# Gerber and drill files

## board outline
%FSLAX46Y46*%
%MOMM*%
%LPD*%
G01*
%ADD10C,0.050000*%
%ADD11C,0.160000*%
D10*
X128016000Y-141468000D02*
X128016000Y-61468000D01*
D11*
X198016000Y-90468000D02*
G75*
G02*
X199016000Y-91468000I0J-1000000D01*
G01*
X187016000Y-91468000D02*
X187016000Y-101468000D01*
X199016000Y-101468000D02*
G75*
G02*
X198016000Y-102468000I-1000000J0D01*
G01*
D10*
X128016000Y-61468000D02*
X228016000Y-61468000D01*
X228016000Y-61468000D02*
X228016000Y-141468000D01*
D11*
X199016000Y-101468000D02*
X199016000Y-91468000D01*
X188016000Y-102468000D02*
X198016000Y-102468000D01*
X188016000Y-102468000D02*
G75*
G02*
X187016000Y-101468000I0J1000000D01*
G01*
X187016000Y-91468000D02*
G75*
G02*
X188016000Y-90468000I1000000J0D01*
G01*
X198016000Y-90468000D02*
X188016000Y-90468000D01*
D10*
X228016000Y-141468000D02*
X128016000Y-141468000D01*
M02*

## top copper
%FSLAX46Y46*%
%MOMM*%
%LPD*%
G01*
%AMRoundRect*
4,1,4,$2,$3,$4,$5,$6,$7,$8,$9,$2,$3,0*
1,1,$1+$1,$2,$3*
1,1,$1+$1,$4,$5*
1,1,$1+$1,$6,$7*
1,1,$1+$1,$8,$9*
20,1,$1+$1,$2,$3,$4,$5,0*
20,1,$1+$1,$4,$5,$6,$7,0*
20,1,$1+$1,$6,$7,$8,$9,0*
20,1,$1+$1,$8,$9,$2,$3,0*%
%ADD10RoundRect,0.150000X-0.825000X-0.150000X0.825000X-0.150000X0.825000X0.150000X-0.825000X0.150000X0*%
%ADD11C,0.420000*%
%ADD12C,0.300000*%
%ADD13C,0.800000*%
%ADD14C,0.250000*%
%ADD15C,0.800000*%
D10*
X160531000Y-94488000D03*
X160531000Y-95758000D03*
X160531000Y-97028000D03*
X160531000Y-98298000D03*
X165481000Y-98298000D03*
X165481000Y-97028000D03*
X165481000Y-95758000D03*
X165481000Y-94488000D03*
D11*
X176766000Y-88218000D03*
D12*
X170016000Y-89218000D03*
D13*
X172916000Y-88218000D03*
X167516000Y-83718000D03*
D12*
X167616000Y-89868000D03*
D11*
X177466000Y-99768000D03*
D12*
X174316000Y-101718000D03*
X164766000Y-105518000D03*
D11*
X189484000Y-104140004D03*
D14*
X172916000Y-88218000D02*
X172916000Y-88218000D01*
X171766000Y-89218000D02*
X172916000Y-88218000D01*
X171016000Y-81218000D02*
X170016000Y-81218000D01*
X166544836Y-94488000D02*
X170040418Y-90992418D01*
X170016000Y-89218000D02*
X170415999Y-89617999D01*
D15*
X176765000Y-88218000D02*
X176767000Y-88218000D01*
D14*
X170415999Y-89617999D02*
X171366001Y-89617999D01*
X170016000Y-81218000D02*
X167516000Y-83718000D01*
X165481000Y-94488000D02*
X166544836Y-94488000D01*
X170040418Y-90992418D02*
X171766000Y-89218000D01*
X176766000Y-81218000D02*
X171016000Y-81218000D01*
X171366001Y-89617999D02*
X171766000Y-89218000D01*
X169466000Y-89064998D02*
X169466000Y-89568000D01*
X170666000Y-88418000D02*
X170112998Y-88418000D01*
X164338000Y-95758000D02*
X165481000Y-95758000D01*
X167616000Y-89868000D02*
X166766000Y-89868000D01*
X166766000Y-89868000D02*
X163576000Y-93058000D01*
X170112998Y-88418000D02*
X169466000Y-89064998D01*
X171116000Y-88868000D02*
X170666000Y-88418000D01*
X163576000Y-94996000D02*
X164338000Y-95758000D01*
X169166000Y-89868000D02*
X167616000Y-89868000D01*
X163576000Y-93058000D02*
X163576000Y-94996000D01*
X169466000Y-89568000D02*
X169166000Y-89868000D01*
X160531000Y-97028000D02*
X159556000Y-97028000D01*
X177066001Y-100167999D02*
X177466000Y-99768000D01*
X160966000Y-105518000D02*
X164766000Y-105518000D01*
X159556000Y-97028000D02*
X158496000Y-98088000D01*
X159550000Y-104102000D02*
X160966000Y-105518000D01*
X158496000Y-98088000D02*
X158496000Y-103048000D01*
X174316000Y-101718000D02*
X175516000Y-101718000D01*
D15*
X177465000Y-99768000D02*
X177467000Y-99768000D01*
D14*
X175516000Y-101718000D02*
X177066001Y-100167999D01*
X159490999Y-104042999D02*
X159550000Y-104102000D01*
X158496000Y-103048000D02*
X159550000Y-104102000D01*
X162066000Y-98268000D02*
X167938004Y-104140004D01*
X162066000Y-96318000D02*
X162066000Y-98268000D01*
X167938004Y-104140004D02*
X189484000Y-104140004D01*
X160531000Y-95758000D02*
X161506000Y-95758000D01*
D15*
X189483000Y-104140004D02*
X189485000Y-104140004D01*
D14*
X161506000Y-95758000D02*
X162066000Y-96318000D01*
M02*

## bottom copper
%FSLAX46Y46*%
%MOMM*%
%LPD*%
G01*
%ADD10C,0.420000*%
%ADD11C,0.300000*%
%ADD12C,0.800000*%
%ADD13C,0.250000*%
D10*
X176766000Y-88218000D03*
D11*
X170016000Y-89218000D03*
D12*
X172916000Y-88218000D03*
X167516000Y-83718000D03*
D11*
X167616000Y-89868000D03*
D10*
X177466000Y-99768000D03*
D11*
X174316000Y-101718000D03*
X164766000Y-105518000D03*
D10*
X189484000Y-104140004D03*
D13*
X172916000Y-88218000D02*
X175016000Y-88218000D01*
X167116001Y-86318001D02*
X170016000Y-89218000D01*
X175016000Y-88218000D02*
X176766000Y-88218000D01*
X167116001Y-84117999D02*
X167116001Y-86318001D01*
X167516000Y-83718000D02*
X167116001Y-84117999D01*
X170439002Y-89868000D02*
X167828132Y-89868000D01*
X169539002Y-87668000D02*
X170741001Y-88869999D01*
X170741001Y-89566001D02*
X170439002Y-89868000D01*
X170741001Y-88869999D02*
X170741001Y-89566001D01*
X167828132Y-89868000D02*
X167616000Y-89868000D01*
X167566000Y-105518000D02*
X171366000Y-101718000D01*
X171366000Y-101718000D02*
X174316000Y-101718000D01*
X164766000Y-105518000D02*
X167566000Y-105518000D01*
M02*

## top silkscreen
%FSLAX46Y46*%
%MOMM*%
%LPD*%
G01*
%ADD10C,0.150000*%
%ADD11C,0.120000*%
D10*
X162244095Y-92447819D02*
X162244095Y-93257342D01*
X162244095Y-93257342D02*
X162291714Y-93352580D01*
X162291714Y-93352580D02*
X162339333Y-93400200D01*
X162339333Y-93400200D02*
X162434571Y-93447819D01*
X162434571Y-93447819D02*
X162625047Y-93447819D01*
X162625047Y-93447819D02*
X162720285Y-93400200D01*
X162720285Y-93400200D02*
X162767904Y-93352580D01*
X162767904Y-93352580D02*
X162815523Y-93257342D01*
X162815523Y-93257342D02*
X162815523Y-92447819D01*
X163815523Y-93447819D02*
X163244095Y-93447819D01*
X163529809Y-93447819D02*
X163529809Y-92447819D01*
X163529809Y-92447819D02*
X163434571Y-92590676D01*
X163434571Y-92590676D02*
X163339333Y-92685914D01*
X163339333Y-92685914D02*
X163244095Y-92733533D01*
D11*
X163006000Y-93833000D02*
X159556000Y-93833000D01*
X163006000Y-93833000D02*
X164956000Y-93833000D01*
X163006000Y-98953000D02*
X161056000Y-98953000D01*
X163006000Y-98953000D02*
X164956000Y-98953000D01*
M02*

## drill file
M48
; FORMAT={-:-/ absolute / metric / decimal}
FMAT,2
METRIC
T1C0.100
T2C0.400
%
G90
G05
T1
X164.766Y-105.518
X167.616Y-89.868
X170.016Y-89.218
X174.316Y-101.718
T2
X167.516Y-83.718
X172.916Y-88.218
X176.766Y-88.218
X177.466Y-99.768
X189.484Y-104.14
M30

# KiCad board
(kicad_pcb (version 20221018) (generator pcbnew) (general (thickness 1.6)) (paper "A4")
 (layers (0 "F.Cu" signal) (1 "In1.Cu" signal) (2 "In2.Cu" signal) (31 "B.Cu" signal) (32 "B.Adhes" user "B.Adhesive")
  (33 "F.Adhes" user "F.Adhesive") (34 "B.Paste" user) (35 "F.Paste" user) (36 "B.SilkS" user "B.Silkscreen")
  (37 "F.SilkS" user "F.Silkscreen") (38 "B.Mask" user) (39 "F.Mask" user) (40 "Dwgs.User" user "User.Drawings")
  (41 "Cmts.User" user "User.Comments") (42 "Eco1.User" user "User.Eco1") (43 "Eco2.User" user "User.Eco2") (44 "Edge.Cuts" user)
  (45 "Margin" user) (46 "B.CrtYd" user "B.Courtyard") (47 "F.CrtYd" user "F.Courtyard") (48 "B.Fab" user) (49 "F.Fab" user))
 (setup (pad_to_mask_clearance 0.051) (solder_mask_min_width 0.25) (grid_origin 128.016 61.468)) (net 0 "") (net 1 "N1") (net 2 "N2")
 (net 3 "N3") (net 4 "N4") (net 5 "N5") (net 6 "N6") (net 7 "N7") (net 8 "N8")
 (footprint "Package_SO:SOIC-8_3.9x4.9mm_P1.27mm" (layer "F.Cu") (at 163.006 96.393)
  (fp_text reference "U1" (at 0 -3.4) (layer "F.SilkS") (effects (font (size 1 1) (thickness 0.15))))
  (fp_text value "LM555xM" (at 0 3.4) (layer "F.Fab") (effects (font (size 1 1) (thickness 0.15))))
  (fp_line (start 0 -2.56) (end -3.45 -2.56) (stroke (width 0.12) (type solid)) (layer "F.SilkS"))
  (fp_line (start 0 -2.56) (end 1.95 -2.56) (stroke (width 0.12) (type solid)) (layer "F.SilkS"))
  (fp_line (start 0 2.56) (end -1.95 2.56) (stroke (width 0.12) (type solid)) (layer "F.SilkS"))
  (fp_line (start 0 2.56) (end 1.95 2.56) (stroke (width 0.12) (type solid)) (layer "F.SilkS"))
  (pad "1" smd roundrect (at -2.475 -1.905) (size 1.95 0.6) (layers "F.Cu" "F.Paste" "F.Mask") (roundrect_rratio 0.25) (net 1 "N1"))
  (pad "2" smd roundrect (at -2.475 -0.635) (size 1.95 0.6) (layers "F.Cu" "F.Paste" "F.Mask") (roundrect_rratio 0.25) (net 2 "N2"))
  (pad "3" smd roundrect (at -2.475 0.635) (size 1.95 0.6) (layers "F.Cu" "F.Paste" "F.Mask") (roundrect_rratio 0.25) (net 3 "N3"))
  (pad "4" smd roundrect (at -2.475 1.905) (size 1.95 0.6) (layers "F.Cu" "F.Paste" "F.Mask") (roundrect_rratio 0.25) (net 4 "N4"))
  (pad "5" smd roundrect (at 2.475 1.905) (size 1.95 0.6) (layers "F.Cu" "F.Paste" "F.Mask") (roundrect_rratio 0.25) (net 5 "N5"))
  (pad "6" smd roundrect (at 2.475 0.635) (size 1.95 0.6) (layers "F.Cu" "F.Paste" "F.Mask") (roundrect_rratio 0.25) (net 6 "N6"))
  (pad "7" smd roundrect (at 2.475 -0.635) (size 1.95 0.6) (layers "F.Cu" "F.Paste" "F.Mask") (roundrect_rratio 0.25) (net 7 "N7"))
  (pad "8" smd roundrect (at 2.475 -1.905) (size 1.95 0.6) (layers "F.Cu" "F.Paste" "F.Mask") (roundrect_rratio 0.25) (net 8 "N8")))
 (gr_line (start 128.016 141.468) (end 128.016 61.468) (stroke (width 0.05) (type solid)) (layer "Edge.Cuts"))
 (gr_arc (start 198.016 90.468) (mid 198.723107 90.760893) (end 199.016 91.468) (stroke (width 0.16) (type solid)) (layer "Edge.Cuts"))
 (gr_line (start 187.016 91.468) (end 187.016 101.468) (stroke (width 0.16) (type solid)) (layer "Edge.Cuts"))
 (gr_arc (start 199.016 101.468) (mid 198.723107 102.175107) (end 198.016 102.468) (stroke (width 0.16) (type solid)) (layer "Edge.Cuts"))
 (gr_line (start 128.016 61.468) (end 228.016 61.468) (stroke (width 0.05) (type solid)) (layer "Edge.Cuts"))
 (gr_line (start 228.016 61.468) (end 228.016 141.468) (stroke (width 0.05) (type solid)) (layer "Edge.Cuts"))
 (gr_line (start 199.016 101.468) (end 199.016 91.468) (stroke (width 0.16) (type solid)) (layer "Edge.Cuts"))
 (gr_line (start 188.016 102.468) (end 198.016 102.468) (stroke (width 0.16) (type solid)) (layer "Edge.Cuts"))
 (gr_arc (start 188.016 102.468) (mid 187.308893 102.175107) (end 187.016 101.468) (stroke (width 0.16) (type solid)) (layer "Edge.Cuts"))
 (gr_arc (start 187.016 91.468) (mid 187.308893 90.760893) (end 188.016 90.468) (stroke (width 0.16) (type solid)) (layer "Edge.Cuts"))
 (gr_line (start 198.016 90.468) (end 188.016 90.468) (stroke (width 0.16) (type solid)) (layer "Edge.Cuts"))
 (gr_line (start 228.016 141.468) (end 128.016 141.468) (stroke (width 0.05) (type solid)) (layer "Edge.Cuts"))
 (segment (start 172.916 88.218) (end 172.916 88.218) (width 0.25) (layer "F.Cu") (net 8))
 (segment (start 171.766 89.218) (end 172.916 88.218) (width 0.25) (layer "F.Cu") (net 8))
 (segment (start 171.016 81.218) (end 170.016 81.218) (width 0.25) (layer "F.Cu") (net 8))
 (segment (start 166.544836 94.488) (end 170.040418 90.992418) (width 0.25) (layer "F.Cu") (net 8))
 (segment (start 170.016 89.218) (end 170.415999 89.617999) (width 0.25) (layer "F.Cu") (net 8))
 (segment (start 176.765 88.218) (end 176.767 88.218) (width 0.8) (layer "F.Cu") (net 8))
 (segment (start 170.415999 89.617999) (end 171.366001 89.617999) (width 0.25) (layer "F.Cu") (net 8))
 (segment (start 170.016 81.218) (end 167.516 83.718) (width 0.25) (layer "F.Cu") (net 8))
 (segment (start 165.481 94.488) (end 166.544836 94.488) (width 0.25) (layer "F.Cu") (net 8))
 (segment (start 170.040418 90.992418) (end 171.766 89.218) (width 0.25) (layer "F.Cu") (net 8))
 (segment (start 176.766 81.218) (end 171.016 81.218) (width 0.25) (layer "F.Cu") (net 8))
 (segment (start 171.366001 89.617999) (end 171.766 89.218) (width 0.25) (layer "F.Cu") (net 8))
 (via (at 176.766 88.218) (size 0.42) (drill 0.4) (layers "F.Cu" "B.Cu") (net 8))
 (segment (start 172.916 88.218) (end 175.016 88.218) (width 0.25) (layer "B.Cu") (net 8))
 (segment (start 167.116001 86.318001) (end 170.016 89.218) (width 0.25) (layer "B.Cu") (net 8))
 (segment (start 175.016 88.218) (end 176.766 88.218) (width 0.25) (layer "B.Cu") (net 8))
 (segment (start 167.116001 84.117999) (end 167.116001 86.318001) (width 0.25) (layer "B.Cu") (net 8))
 (segment (start 167.516 83.718) (end 167.116001 84.117999) (width 0.25) (layer "B.Cu") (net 8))
 (via (at 170.016 89.218) (size 0.3) (drill 0.1) (layers "F.Cu" "B.Cu") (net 8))
 (via (at 172.916 88.218) (size 0.8) (drill 0.4) (layers "F.Cu" "B.Cu") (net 8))
 (via (at 167.516 83.718) (size 0.8) (drill 0.4) (layers "F.Cu" "B.Cu") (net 8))
 (segment (start 169.466 89.064998) (end 169.466 89.568) (width 0.25) (layer "F.Cu") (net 7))
 (segment (start 170.666 88.418) (end 170.112998 88.418) (width 0.25) (layer "F.Cu") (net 7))
 (segment (start 164.338 95.758) (end 165.481 95.758) (width 0.25) (layer "F.Cu") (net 7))
 (segment (start 167.616 89.868) (end 166.766 89.868) (width 0.25) (layer "F.Cu") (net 7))
 (segment (start 166.766 89.868) (end 163.576 93.058) (width 0.25) (layer "F.Cu") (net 7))
 (segment (start 170.112998 88.418) (end 169.466 89.064998) (width 0.25) (layer "F.Cu") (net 7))
 (segment (start 171.116 88.868) (end 170.666 88.418) (width 0.25) (layer "F.Cu") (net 7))
 (segment (start 163.576 94.996) (end 164.338 95.758) (width 0.25) (layer "F.Cu") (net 7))
 (segment (start 169.166 89.868) (end 167.616 89.868) (width 0.25) (layer "F.Cu") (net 7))
 (segment (start 163.576 93.058) (end 163.576 94.996) (width 0.25) (layer "F.Cu") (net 7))
 (segment (start 169.466 89.568) (end 169.166 89.868) (width 0.25) (layer "F.Cu") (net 7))
 (segment (start 170.439002 89.868) (end 167.828132 89.868) (width 0.25) (layer "B.Cu") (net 7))
 (segment (start 169.539002 87.668) (end 170.741001 88.869999) (width 0.25) (layer "B.Cu") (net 7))
 (segment (start 170.741001 89.566001) (end 170.439002 89.868) (width 0.25) (layer "B.Cu") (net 7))
 (segment (start 170.741001 88.869999) (end 170.741001 89.566001) (width 0.25) (layer "B.Cu") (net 7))
 (segment (start 167.828132 89.868) (end 167.616 89.868) (width 0.25) (layer "B.Cu") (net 7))
 (via (at 167.616 89.868) (size 0.3) (drill 0.1) (layers "F.Cu" "B.Cu") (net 7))
 (segment (start 160.531 97.028) (end 159.556 97.028) (width 0.25) (layer "F.Cu") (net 3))
 (segment (start 177.066001 100.167999) (end 177.466 99.768) (width 0.25) (layer "F.Cu") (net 3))
 (segment (start 160.966 105.518) (end 164.766 105.518) (width 0.25) (layer "F.Cu") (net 3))
 (segment (start 159.556 97.028) (end 158.496 98.088) (width 0.25) (layer "F.Cu") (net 3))
 (segment (start 159.55 104.102) (end 160.966 105.518) (width 0.25) (layer "F.Cu") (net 3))
 (segment (start 158.496 98.088) (end 158.496 103.048) (width 0.25) (layer "F.Cu") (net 3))
 (segment (start 174.316 101.718) (end 175.516 101.718) (width 0.25) (layer "F.Cu") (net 3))
 (segment (start 177.465 99.768) (end 177.467 99.768) (width 0.8) (layer "F.Cu") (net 3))
 (segment (start 175.516 101.718) (end 177.066001 100.167999) (width 0.25) (layer "F.Cu") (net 3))
 (segment (start 159.490999 104.042999) (end 159.55 104.102) (width 0.25) (layer "F.Cu") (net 3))
 (segment (start 158.496 103.048) (end 159.55 104.102) (width 0.25) (layer "F.Cu") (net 3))
 (via (at 177.466 99.768) (size 0.42) (drill 0.4) (layers "F.Cu" "B.Cu") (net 3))
 (segment (start 167.566 105.518) (end 171.366 101.718) (width 0.25) (layer "B.Cu") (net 3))
 (segment (start 171.366 101.718) (end 174.316 101.718) (width 0.25) (layer "B.Cu") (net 3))
 (segment (start 164.766 105.518) (end 167.566 105.518) (width 0.25) (layer "B.Cu") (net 3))
 (via (at 174.316 101.718) (size 0.3) (drill 0.1) (layers "F.Cu" "B.Cu") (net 3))
 (via (at 164.766 105.518) (size 0.3) (drill 0.1) (layers "F.Cu" "B.Cu") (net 3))
 (segment (start 162.066 98.268) (end 167.938004 104.140004) (width 0.25) (layer "F.Cu") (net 2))
 (segment (start 162.066 96.318) (end 162.066 98.268) (width 0.25) (layer "F.Cu") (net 2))
 (segment (start 167.938004 104.140004) (end 189.484 104.140004) (width 0.25) (layer "F.Cu") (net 2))
 (segment (start 160.531 95.758) (end 161.506 95.758) (width 0.25) (layer "F.Cu") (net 2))
 (segment (start 189.483 104.140004) (end 189.485 104.140004) (width 0.8) (layer "F.Cu") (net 2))
 (segment (start 161.506 95.758) (end 162.066 96.318) (width 0.25) (layer "F.Cu") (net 2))
 (via (at 189.484 104.140004) (size 0.42) (drill 0.4) (layers "F.Cu" "B.Cu") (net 2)))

